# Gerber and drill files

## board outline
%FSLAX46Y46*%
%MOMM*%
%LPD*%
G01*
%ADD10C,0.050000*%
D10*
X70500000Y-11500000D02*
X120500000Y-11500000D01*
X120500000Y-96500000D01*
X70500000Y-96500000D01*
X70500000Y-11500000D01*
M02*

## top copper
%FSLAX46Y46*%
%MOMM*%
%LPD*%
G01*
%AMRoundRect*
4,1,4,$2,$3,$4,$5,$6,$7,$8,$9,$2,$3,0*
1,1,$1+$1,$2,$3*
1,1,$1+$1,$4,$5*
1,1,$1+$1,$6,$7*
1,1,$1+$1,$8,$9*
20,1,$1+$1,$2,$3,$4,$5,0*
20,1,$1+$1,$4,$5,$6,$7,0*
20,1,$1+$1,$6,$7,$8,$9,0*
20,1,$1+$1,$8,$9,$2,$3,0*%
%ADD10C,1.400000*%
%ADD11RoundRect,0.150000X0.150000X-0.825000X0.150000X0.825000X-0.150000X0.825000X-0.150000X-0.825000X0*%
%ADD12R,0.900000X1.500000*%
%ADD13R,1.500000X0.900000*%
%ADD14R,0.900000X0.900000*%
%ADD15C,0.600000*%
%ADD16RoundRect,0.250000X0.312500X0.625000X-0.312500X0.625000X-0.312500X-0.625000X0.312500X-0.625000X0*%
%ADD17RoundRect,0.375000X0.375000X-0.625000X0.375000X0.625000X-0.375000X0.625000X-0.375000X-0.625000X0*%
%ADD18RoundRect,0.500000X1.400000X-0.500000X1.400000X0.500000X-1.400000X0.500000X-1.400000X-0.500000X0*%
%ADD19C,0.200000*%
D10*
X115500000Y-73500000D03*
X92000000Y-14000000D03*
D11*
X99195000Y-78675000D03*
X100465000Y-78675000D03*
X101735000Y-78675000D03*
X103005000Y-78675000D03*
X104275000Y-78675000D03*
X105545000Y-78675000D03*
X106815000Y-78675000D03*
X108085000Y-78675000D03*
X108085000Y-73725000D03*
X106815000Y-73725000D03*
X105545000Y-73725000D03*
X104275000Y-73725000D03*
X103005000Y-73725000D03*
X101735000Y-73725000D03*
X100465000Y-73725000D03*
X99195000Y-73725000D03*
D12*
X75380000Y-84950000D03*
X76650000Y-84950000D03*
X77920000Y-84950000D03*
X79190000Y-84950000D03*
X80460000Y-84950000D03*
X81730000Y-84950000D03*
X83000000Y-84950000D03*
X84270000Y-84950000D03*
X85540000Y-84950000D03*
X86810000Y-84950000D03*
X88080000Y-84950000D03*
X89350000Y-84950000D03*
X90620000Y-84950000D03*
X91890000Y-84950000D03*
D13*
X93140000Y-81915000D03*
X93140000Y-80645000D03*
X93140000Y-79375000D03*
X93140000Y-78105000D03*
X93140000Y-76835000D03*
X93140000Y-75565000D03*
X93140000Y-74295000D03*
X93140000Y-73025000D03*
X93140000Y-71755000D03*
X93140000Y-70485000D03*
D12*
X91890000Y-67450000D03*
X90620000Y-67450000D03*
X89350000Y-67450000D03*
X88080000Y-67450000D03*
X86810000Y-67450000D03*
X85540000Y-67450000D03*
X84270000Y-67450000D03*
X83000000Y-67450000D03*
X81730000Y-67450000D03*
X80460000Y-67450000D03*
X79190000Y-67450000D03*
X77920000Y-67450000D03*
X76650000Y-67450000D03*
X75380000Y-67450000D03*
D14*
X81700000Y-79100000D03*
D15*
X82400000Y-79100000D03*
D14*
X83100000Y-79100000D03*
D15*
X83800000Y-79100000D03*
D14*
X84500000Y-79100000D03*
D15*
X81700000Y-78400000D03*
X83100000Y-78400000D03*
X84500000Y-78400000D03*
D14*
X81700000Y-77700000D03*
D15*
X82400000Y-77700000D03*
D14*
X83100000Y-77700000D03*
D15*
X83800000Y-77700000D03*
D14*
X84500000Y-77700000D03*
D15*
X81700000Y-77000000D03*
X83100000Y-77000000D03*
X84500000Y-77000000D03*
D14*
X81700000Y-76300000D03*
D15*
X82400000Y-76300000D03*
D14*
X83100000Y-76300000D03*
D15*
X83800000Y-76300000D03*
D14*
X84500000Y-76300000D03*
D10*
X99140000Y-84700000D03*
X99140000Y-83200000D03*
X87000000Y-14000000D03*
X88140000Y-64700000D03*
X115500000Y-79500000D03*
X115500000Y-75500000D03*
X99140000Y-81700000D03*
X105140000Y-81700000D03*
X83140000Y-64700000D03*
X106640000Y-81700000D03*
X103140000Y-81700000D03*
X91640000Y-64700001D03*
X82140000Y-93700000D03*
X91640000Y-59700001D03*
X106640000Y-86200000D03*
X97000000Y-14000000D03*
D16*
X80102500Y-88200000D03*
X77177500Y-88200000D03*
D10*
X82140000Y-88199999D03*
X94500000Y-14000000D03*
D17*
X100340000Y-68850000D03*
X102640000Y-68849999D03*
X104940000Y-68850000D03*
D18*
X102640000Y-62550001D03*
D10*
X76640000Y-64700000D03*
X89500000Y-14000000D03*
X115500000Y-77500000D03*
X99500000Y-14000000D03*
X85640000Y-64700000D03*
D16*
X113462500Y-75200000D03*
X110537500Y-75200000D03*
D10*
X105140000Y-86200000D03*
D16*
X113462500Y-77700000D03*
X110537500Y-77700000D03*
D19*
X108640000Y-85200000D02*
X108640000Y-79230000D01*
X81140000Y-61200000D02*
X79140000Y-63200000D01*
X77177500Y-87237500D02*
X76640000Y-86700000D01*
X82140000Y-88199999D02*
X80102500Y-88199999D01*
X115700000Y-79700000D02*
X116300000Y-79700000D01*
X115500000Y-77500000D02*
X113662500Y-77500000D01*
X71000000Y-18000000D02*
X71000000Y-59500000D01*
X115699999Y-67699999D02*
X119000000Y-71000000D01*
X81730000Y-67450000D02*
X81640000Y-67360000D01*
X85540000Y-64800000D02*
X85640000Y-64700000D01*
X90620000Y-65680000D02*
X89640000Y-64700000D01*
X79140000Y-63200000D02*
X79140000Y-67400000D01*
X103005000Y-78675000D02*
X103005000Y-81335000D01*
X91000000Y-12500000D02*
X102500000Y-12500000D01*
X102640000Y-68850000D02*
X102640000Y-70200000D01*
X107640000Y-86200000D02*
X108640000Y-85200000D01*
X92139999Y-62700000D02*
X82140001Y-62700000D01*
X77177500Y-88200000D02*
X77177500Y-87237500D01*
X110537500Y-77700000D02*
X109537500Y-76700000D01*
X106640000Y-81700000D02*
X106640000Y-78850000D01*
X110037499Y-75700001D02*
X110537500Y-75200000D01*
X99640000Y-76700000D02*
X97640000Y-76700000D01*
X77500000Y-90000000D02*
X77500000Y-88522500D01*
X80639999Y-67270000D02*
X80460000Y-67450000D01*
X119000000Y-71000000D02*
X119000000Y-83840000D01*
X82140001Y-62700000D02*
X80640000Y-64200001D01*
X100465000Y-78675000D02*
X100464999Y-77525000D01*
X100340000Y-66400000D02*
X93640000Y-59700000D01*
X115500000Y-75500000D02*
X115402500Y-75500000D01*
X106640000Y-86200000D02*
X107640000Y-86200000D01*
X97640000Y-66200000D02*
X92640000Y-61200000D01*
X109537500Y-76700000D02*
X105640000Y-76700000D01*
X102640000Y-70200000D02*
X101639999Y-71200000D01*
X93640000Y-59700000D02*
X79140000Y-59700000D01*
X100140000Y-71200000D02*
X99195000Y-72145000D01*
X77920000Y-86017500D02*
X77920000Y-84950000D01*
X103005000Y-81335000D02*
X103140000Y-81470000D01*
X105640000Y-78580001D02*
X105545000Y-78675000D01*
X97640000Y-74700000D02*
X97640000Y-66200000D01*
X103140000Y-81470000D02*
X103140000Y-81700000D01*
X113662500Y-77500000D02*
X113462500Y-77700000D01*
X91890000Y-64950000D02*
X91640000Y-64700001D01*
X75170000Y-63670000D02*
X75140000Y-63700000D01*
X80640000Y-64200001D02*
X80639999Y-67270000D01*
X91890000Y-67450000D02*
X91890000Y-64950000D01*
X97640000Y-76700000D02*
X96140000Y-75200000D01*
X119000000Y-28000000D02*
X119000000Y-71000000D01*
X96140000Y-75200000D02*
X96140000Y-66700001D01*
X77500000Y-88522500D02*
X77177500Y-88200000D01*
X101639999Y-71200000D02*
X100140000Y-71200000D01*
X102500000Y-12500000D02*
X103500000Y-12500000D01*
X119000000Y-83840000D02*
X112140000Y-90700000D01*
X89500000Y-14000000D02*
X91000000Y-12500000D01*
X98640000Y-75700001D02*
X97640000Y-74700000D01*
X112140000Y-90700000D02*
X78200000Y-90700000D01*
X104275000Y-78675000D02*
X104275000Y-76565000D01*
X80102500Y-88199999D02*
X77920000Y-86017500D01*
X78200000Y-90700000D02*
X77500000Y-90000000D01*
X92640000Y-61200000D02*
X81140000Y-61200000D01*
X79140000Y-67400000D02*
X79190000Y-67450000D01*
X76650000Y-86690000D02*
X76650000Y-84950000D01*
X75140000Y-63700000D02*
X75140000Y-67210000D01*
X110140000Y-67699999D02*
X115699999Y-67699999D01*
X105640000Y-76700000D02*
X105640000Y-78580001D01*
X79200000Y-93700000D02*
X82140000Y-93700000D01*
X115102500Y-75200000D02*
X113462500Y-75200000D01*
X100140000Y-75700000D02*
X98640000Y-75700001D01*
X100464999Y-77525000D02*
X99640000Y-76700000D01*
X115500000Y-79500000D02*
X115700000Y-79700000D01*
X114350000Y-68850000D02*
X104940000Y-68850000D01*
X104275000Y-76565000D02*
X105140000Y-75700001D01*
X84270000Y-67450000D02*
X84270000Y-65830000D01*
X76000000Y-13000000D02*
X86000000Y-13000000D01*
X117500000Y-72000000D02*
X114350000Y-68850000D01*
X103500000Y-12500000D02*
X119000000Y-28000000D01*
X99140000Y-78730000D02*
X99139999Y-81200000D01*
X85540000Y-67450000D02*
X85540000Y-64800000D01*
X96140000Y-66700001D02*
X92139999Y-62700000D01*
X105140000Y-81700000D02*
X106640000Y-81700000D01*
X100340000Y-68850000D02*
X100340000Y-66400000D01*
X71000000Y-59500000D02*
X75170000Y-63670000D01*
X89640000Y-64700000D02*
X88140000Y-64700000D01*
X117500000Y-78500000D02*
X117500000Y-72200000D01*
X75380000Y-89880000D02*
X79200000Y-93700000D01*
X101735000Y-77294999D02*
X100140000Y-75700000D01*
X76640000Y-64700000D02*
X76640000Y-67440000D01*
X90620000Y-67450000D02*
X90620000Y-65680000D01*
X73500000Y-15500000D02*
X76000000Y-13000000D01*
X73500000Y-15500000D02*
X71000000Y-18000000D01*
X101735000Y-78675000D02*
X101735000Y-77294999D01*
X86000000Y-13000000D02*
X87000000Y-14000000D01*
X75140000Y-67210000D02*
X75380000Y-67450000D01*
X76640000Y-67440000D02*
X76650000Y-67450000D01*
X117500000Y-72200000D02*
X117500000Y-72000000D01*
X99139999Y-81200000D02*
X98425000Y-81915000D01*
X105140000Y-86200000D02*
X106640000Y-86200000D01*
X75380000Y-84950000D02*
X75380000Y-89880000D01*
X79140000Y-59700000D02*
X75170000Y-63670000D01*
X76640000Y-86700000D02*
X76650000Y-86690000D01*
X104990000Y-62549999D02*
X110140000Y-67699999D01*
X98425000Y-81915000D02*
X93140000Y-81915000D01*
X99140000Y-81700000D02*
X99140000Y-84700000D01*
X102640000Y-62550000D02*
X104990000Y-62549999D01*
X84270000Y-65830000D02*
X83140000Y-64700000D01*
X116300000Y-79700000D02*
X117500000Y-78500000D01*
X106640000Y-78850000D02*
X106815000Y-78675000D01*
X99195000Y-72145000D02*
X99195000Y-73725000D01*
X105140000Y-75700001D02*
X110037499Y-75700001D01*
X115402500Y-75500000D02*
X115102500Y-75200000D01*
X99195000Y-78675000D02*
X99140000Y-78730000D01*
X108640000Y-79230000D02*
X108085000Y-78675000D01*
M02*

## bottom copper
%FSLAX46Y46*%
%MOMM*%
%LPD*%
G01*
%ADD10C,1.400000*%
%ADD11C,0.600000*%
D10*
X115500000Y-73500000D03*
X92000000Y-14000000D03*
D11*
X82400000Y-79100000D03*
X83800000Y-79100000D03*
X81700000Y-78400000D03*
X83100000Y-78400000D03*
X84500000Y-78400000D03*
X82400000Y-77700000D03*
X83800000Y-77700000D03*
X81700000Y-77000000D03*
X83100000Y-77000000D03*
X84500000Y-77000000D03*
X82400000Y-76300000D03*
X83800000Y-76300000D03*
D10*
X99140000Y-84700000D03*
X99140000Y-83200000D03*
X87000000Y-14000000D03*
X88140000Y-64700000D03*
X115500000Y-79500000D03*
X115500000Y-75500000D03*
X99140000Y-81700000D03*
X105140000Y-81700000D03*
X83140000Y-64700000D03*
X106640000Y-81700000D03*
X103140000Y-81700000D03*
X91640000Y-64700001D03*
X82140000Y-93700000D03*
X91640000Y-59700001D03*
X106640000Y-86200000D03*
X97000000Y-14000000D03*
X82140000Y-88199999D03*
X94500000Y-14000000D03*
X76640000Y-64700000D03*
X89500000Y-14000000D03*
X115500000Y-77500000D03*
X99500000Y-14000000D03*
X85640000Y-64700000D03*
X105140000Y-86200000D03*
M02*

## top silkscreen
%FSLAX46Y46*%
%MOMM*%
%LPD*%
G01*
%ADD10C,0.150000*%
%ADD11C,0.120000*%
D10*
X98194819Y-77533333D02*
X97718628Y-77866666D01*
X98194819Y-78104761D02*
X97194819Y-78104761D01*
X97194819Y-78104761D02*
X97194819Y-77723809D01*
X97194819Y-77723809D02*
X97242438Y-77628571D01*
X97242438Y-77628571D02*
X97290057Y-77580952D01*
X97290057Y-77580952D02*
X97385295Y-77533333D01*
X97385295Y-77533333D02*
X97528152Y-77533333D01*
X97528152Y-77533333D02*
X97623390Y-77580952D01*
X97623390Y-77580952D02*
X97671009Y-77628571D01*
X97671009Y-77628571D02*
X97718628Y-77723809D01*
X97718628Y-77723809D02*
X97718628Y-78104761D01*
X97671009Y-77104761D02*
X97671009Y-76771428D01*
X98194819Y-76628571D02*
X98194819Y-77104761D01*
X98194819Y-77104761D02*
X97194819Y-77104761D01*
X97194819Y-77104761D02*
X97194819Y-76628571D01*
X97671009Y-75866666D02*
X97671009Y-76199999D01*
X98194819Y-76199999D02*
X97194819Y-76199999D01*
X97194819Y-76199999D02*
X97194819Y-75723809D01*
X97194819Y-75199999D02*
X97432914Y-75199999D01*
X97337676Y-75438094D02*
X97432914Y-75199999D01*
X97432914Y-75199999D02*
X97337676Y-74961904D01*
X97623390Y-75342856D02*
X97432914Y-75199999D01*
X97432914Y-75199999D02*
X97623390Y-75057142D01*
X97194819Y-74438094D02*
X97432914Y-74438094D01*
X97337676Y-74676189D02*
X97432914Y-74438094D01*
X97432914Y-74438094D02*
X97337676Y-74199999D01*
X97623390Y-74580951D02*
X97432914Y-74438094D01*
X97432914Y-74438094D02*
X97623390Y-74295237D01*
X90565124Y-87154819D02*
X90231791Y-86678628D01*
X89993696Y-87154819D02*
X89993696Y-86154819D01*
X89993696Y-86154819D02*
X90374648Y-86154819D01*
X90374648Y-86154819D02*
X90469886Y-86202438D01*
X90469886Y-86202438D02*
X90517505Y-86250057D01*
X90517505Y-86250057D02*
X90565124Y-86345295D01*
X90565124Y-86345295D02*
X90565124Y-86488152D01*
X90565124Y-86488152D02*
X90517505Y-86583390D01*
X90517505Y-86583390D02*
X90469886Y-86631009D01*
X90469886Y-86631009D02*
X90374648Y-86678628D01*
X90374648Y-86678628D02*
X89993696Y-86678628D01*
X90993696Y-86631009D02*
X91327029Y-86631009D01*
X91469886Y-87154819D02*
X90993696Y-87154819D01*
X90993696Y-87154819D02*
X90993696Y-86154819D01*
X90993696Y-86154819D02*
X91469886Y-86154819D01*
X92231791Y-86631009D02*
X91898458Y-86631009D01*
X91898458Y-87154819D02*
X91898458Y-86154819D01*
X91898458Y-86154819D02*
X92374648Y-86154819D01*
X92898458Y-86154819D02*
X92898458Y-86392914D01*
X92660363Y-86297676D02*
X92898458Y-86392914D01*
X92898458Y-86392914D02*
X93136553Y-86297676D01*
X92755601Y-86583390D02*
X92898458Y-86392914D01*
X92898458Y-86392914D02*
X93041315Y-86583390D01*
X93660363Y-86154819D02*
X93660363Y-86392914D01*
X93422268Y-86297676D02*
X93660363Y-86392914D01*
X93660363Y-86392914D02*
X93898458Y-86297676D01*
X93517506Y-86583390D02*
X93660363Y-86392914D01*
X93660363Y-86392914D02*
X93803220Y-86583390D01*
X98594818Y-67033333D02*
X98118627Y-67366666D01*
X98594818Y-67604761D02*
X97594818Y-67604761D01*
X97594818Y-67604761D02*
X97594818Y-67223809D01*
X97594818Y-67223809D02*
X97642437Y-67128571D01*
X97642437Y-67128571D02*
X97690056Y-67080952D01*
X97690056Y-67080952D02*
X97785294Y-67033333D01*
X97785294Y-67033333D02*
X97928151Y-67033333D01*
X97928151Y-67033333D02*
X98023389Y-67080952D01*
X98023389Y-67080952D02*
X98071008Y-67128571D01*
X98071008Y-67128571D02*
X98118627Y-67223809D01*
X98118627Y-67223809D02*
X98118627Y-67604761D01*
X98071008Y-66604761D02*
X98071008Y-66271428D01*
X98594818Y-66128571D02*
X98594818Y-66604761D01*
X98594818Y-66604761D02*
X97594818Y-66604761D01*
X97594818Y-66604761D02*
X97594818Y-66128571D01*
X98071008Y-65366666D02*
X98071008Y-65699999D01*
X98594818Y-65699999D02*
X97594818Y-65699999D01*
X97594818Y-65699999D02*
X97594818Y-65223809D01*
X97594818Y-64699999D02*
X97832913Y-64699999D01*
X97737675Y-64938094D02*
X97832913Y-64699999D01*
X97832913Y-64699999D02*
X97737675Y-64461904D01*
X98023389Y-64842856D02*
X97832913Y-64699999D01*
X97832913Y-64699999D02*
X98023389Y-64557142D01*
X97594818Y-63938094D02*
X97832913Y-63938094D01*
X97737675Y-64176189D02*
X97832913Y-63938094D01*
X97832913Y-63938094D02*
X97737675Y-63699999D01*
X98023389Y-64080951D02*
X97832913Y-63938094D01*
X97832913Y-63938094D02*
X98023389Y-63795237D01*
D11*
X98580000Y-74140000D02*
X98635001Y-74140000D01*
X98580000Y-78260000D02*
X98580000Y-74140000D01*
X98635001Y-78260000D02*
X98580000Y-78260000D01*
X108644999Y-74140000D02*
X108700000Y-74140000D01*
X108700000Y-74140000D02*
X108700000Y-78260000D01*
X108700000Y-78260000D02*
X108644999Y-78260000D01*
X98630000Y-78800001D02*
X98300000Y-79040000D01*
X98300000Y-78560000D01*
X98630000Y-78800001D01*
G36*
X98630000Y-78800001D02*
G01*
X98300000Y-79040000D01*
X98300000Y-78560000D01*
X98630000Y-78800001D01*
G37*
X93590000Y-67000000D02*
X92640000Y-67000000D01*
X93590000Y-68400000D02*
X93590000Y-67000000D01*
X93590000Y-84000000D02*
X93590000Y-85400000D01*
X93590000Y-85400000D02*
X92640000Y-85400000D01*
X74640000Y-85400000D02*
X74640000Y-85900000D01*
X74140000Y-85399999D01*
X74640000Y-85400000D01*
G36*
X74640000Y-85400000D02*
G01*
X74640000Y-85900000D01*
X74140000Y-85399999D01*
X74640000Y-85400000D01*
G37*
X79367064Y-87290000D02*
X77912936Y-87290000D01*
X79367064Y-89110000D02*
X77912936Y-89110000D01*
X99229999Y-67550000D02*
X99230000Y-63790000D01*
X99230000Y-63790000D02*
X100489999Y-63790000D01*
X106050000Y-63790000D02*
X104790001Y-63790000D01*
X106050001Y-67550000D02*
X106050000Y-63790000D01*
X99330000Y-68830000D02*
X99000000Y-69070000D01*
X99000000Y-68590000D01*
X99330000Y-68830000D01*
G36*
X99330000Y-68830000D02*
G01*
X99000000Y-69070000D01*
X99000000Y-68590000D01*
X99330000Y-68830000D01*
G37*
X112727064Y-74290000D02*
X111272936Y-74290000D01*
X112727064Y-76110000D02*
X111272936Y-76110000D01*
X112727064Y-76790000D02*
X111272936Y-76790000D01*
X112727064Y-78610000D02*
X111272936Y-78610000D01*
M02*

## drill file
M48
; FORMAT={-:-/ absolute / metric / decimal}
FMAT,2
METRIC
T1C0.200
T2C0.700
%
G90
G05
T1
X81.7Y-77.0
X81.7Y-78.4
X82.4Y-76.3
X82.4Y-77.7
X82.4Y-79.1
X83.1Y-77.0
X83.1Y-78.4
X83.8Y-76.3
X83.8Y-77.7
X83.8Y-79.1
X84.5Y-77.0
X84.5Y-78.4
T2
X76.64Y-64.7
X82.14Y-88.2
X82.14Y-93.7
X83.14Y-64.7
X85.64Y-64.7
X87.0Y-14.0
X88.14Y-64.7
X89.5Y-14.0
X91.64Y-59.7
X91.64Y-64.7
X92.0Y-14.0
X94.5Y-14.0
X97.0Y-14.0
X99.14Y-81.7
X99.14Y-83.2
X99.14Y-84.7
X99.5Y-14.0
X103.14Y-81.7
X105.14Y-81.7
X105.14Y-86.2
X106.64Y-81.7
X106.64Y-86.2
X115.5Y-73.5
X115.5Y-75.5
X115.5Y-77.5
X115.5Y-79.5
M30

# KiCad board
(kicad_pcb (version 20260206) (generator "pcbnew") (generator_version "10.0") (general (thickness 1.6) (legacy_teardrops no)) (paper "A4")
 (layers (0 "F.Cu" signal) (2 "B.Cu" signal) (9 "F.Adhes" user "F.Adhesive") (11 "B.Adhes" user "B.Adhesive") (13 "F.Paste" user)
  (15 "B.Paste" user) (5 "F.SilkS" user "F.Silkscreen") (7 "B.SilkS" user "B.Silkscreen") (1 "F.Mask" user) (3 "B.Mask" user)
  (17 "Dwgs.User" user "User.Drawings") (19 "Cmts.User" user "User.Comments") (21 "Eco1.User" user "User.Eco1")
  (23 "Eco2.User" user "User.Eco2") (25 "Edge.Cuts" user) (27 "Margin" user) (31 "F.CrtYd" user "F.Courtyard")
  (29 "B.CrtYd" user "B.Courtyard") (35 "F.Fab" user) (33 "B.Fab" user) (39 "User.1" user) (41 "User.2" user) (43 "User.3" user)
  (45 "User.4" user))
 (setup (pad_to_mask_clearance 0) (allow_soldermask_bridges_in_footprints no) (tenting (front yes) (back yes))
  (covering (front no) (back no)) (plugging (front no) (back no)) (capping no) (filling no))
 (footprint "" (layer "F.Cu") (at 115.5 73.5 90)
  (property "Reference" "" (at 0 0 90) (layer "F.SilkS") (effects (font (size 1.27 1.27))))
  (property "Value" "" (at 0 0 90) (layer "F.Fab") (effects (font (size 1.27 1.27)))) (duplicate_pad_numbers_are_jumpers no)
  (pad "4" thru_hole circle (at 0 0 90) (size 1.4 1.4) (drill 0.7) (layers "*.Cu" "*.Mask") (remove_unused_layers no)))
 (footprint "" (layer "F.Cu") (at 92 14)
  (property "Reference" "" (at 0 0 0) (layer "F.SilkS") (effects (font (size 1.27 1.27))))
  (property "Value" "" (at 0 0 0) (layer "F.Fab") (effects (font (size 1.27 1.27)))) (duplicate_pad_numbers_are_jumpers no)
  (pad "4" thru_hole circle (at 0 0) (size 1.4 1.4) (drill 0.7) (layers "*.Cu" "*.Mask") (remove_unused_layers no)))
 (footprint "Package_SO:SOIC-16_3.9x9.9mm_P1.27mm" (layer "F.Cu") (at 103.64 76.2 90)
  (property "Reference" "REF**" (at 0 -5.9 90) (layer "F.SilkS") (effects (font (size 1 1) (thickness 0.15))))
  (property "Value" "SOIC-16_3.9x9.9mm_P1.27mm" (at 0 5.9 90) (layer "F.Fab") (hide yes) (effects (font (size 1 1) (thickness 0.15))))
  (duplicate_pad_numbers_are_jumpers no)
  (fp_line (start 2.06 -5.06) (end 2.06 -5.004999) (stroke (width 0.12) (type solid)) (layer "F.SilkS"))
  (fp_line (start -2.06 -5.06) (end 2.06 -5.06) (stroke (width 0.12) (type solid)) (layer "F.SilkS"))
  (fp_line (start -2.06 -5.004999) (end -2.06 -5.06) (stroke (width 0.12) (type solid)) (layer "F.SilkS"))
  (fp_line (start 2.06 5.004999) (end 2.06 5.06) (stroke (width 0.12) (type solid)) (layer "F.SilkS"))
  (fp_line (start 2.06 5.06) (end -2.06 5.06) (stroke (width 0.12) (type solid)) (layer "F.SilkS"))
  (fp_line (start -2.06 5.06) (end -2.06 5.004999) (stroke (width 0.12) (type solid)) (layer "F.SilkS"))
  (fp_poly (pts (xy -2.600001 -5.01) (xy -2.84 -5.34) (xy -2.36 -5.34)) (stroke (width 0.12) (type solid)) (fill yes) (layer "F.SilkS"))
  (pad "1" smd roundrect (at -2.475 -4.445 90) (size 1.95 0.6) (layers "F.Cu" "F.Mask" "F.Paste") (roundrect_rratio 0.25))
  (pad "2" smd roundrect (at -2.475 -3.175 90) (size 1.95 0.6) (layers "F.Cu" "F.Mask" "F.Paste") (roundrect_rratio 0.25))
  (pad "3" smd roundrect (at -2.475 -1.905 90) (size 1.95 0.6) (layers "F.Cu" "F.Mask" "F.Paste") (roundrect_rratio 0.25))
  (pad "4" smd roundrect (at -2.475 -0.635 90) (size 1.95 0.6) (layers "F.Cu" "F.Mask" "F.Paste") (roundrect_rratio 0.25))
  (pad "5" smd roundrect (at -2.475 0.635 90) (size 1.95 0.6) (layers "F.Cu" "F.Mask" "F.Paste") (roundrect_rratio 0.25))
  (pad "6" smd roundrect (at -2.475 1.905 90) (size 1.95 0.6) (layers "F.Cu" "F.Mask" "F.Paste") (roundrect_rratio 0.25))
  (pad "7" smd roundrect (at -2.475 3.175 90) (size 1.95 0.6) (layers "F.Cu" "F.Mask" "F.Paste") (roundrect_rratio 0.25))
  (pad "8" smd roundrect (at -2.475 4.445 90) (size 1.95 0.6) (layers "F.Cu" "F.Mask" "F.Paste") (roundrect_rratio 0.25))
  (pad "9" smd roundrect (at 2.475 4.445 90) (size 1.95 0.6) (layers "F.Cu" "F.Mask" "F.Paste") (roundrect_rratio 0.25))
  (pad "10" smd roundrect (at 2.475 3.175 90) (size 1.95 0.6) (layers "F.Cu" "F.Mask" "F.Paste") (roundrect_rratio 0.25))
  (pad "11" smd roundrect (at 2.475 1.905 90) (size 1.95 0.6) (layers "F.Cu" "F.Mask" "F.Paste") (roundrect_rratio 0.25))
  (pad "12" smd roundrect (at 2.475 0.635 90) (size 1.95 0.6) (layers "F.Cu" "F.Mask" "F.Paste") (roundrect_rratio 0.25))
  (pad "13" smd roundrect (at 2.475 -0.635 90) (size 1.95 0.6) (layers "F.Cu" "F.Mask" "F.Paste") (roundrect_rratio 0.25))
  (pad "14" smd roundrect (at 2.475 -1.905 90) (size 1.95 0.6) (layers "F.Cu" "F.Mask" "F.Paste") (roundrect_rratio 0.25))
  (pad "15" smd roundrect (at 2.475 -3.175 90) (size 1.95 0.6) (layers "F.Cu" "F.Mask" "F.Paste") (roundrect_rratio 0.25))
  (pad "16" smd roundrect (at 2.475 -4.445 90) (size 1.95 0.6) (layers "F.Cu" "F.Mask" "F.Paste") (roundrect_rratio 0.25)))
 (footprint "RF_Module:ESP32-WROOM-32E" (layer "F.Cu") (at 80.64 76.2 90)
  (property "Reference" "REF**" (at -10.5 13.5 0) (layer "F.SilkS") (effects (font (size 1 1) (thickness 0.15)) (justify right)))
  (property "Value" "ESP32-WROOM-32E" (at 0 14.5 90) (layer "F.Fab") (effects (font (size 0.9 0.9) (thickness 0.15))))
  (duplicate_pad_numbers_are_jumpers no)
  (fp_line (start 9.2 12.95) (end 9.2 12) (stroke (width 0.12) (type solid)) (layer "F.SilkS"))
  (fp_line (start 7.8 12.95) (end 9.2 12.95) (stroke (width 0.12) (type solid)) (layer "F.SilkS"))
  (fp_line (start -7.8 12.95) (end -9.2 12.95) (stroke (width 0.12) (type solid)) (layer "F.SilkS"))
  (fp_line (start -9.2 12.95) (end -9.2 12) (stroke (width 0.12) (type solid)) (layer "F.SilkS"))
  (fp_poly (pts (xy -9.2 -6) (xy -9.7 -6) (xy -9.199999 -6.5) (xy -9.2 -6)) (stroke (width 0.12) (type solid)) (fill yes) (layer "F.SilkS"))
  (pad "1" smd rect (at -8.75 -5.26 90) (size 1.5 0.9) (layers "F.Cu" "F.Mask" "F.Paste"))
  (pad "2" smd rect (at -8.75 -3.99 90) (size 1.5 0.9) (layers "F.Cu" "F.Mask" "F.Paste"))
  (pad "3" smd rect (at -8.75 -2.72 90) (size 1.5 0.9) (layers "F.Cu" "F.Mask" "F.Paste"))
  (pad "4" smd rect (at -8.75 -1.45 90) (size 1.5 0.9) (layers "F.Cu" "F.Mask" "F.Paste"))
  (pad "5" smd rect (at -8.75 -0.18 90) (size 1.5 0.9) (layers "F.Cu" "F.Mask" "F.Paste"))
  (pad "6" smd rect (at -8.75 1.09 90) (size 1.5 0.9) (layers "F.Cu" "F.Mask" "F.Paste"))
  (pad "7" smd rect (at -8.75 2.36 90) (size 1.5 0.9) (layers "F.Cu" "F.Mask" "F.Paste"))
  (pad "8" smd rect (at -8.75 3.63 90) (size 1.5 0.9) (layers "F.Cu" "F.Mask" "F.Paste"))
  (pad "9" smd rect (at -8.75 4.9 90) (size 1.5 0.9) (layers "F.Cu" "F.Mask" "F.Paste"))
  (pad "10" smd rect (at -8.75 6.17 90) (size 1.5 0.9) (layers "F.Cu" "F.Mask" "F.Paste"))
  (pad "11" smd rect (at -8.75 7.44 90) (size 1.5 0.9) (layers "F.Cu" "F.Mask" "F.Paste"))
  (pad "12" smd rect (at -8.75 8.71 90) (size 1.5 0.9) (layers "F.Cu" "F.Mask" "F.Paste"))
  (pad "13" smd rect (at -8.75 9.98 90) (size 1.5 0.9) (layers "F.Cu" "F.Mask" "F.Paste"))
  (pad "14" smd rect (at -8.75 11.25 90) (size 1.5 0.9) (layers "F.Cu" "F.Mask" "F.Paste"))
  (pad "15" smd rect (at -5.715 12.5 180) (size 1.5 0.9) (layers "F.Cu" "F.Mask" "F.Paste"))
  (pad "16" smd rect (at -4.445 12.5 180) (size 1.5 0.9) (layers "F.Cu" "F.Mask" "F.Paste"))
  (pad "17" smd rect (at -3.175 12.5 180) (size 1.5 0.9) (layers "F.Cu" "F.Mask" "F.Paste"))
  (pad "18" smd rect (at -1.905 12.5 180) (size 1.5 0.9) (layers "F.Cu" "F.Mask" "F.Paste"))
  (pad "19" smd rect (at -0.635 12.5 180) (size 1.5 0.9) (layers "F.Cu" "F.Mask" "F.Paste"))
  (pad "20" smd rect (at 0.635 12.5 180) (size 1.5 0.9) (layers "F.Cu" "F.Mask" "F.Paste"))
  (pad "21" smd rect (at 1.905 12.5 180) (size 1.5 0.9) (layers "F.Cu" "F.Mask" "F.Paste"))
  (pad "22" smd rect (at 3.175 12.5 180) (size 1.5 0.9) (layers "F.Cu" "F.Mask" "F.Paste"))
  (pad "23" smd rect (at 4.445 12.5 180) (size 1.5 0.9) (layers "F.Cu" "F.Mask" "F.Paste"))
  (pad "24" smd rect (at 5.715 12.5 180) (size 1.5 0.9) (layers "F.Cu" "F.Mask" "F.Paste"))
  (pad "25" smd rect (at 8.75 11.25 90) (size 1.5 0.9) (layers "F.Cu" "F.Mask" "F.Paste"))
  (pad "26" smd rect (at 8.75 9.98 90) (size 1.5 0.9) (layers "F.Cu" "F.Mask" "F.Paste"))
  (pad "27" smd rect (at 8.75 8.71 90) (size 1.5 0.9) (layers "F.Cu" "F.Mask" "F.Paste"))
  (pad "28" smd rect (at 8.75 7.44 90) (size 1.5 0.9) (layers "F.Cu" "F.Mask" "F.Paste"))
  (pad "29" smd rect (at 8.75 6.17 90) (size 1.5 0.9) (layers "F.Cu" "F.Mask" "F.Paste"))
  (pad "30" smd rect (at 8.75 4.9 90) (size 1.5 0.9) (layers "F.Cu" "F.Mask" "F.Paste"))
  (pad "31" smd rect (at 8.75 3.63 90) (size 1.5 0.9) (layers "F.Cu" "F.Mask" "F.Paste"))
  (pad "32" smd rect (at 8.75 2.36 90) (size 1.5 0.9) (layers "F.Cu" "F.Mask" "F.Paste"))
  (pad "33" smd rect (at 8.75 1.09 90) (size 1.5 0.9) (layers "F.Cu" "F.Mask" "F.Paste"))
  (pad "34" smd rect (at 8.75 -0.18 90) (size 1.5 0.9) (layers "F.Cu" "F.Mask" "F.Paste"))
  (pad "35" smd rect (at 8.75 -1.45 90) (size 1.5 0.9) (layers "F.Cu" "F.Mask" "F.Paste"))
  (pad "36" smd rect (at 8.75 -2.72 90) (size 1.5 0.9) (layers "F.Cu" "F.Mask" "F.Paste"))
  (pad "37" smd rect (at 8.75 -3.99 90) (size 1.5 0.9) (layers "F.Cu" "F.Mask" "F.Paste"))
  (pad "38" smd rect (at 8.75 -5.26 90) (size 1.5 0.9) (layers "F.Cu" "F.Mask" "F.Paste"))
  (pad "39" smd rect (at -2.9 1.06 90) (size 0.9 0.9) (layers "F.Cu" "F.Mask" "F.Paste") (zone_connect 2))
  (pad "39" thru_hole circle (at -2.9 1.76 90) (size 0.6 0.6) (drill 0.2) (layers "*.Cu" "*.Mask") (remove_unused_layers no)
   (zone_connect 2))
  (pad "39" smd rect (at -2.9 2.46 90) (size 0.9 0.9) (layers "F.Cu" "F.Mask" "F.Paste") (zone_connect 2))
  (pad "39" thru_hole circle (at -2.9 3.16 90) (size 0.6 0.6) (drill 0.2) (layers "*.Cu" "*.Mask") (remove_unused_layers no)
   (zone_connect 2))
  (pad "39" smd rect (at -2.9 3.86 90) (size 0.9 0.9) (layers "F.Cu" "F.Mask" "F.Paste") (zone_connect 2))
  (pad "39" thru_hole circle (at -2.2 1.06 90) (size 0.6 0.6) (drill 0.2) (layers "*.Cu" "*.Mask") (remove_unused_layers no)
   (zone_connect 2))
  (pad "39" thru_hole circle (at -2.2 2.46 90) (size 0.6 0.6) (drill 0.2) (layers "*.Cu" "*.Mask") (remove_unused_layers no)
   (zone_connect 2))
  (pad "39" thru_hole circle (at -2.2 3.86 90) (size 0.6 0.6) (drill 0.2) (layers "*.Cu" "*.Mask") (remove_unused_layers no)
   (zone_connect 2))
  (pad "39" smd rect (at -1.5 1.06 90) (size 0.9 0.9) (layers "F.Cu" "F.Mask" "F.Paste") (zone_connect 2))
  (pad "39" thru_hole circle (at -1.5 1.76 90) (size 0.6 0.6) (drill 0.2) (layers "*.Cu" "*.Mask") (remove_unused_layers no)
   (zone_connect 2))
  (pad "39" smd rect (at -1.5 2.46 90) (size 0.9 0.9) (layers "F.Cu" "F.Mask" "F.Paste") (zone_connect 2))
  (pad "39" thru_hole circle (at -1.5 3.16 90) (size 0.6 0.6) (drill 0.2) (layers "*.Cu" "*.Mask") (remove_unused_layers no)
   (zone_connect 2))
  (pad "39" smd rect (at -1.5 3.86 90) (size 0.9 0.9) (layers "F.Cu" "F.Mask" "F.Paste") (zone_connect 2))
  (pad "39" thru_hole circle (at -0.8 1.06 90) (size 0.6 0.6) (drill 0.2) (layers "*.Cu" "*.Mask") (remove_unused_layers no)
   (zone_connect 2))
  (pad "39" thru_hole circle (at -0.8 2.46 90) (size 0.6 0.6) (drill 0.2) (layers "*.Cu" "*.Mask") (remove_unused_layers no)
   (zone_connect 2))
  (pad "39" thru_hole circle (at -0.8 3.86 90) (size 0.6 0.6) (drill 0.2) (layers "*.Cu" "*.Mask") (remove_unused_layers no)
   (zone_connect 2))
  (pad "39" smd rect (at -0.1 1.06 90) (size 0.9 0.9) (layers "F.Cu" "F.Mask" "F.Paste") (zone_connect 2))
  (pad "39" thru_hole circle (at -0.1 1.76 90) (size 0.6 0.6) (drill 0.2) (layers "*.Cu" "*.Mask") (remove_unused_layers no)
   (zone_connect 2))
  (pad "39" smd rect (at -0.1 2.46 90) (size 0.9 0.9) (layers "F.Cu" "F.Mask" "F.Paste") (zone_connect 2))
  (pad "39" thru_hole circle (at -0.1 3.16 90) (size 0.6 0.6) (drill 0.2) (layers "*.Cu" "*.Mask") (remove_unused_layers no)
   (zone_connect 2))
  (pad "39" smd rect (at -0.1 3.86 90) (size 0.9 0.9) (layers "F.Cu" "F.Mask" "F.Paste") (zone_connect 2))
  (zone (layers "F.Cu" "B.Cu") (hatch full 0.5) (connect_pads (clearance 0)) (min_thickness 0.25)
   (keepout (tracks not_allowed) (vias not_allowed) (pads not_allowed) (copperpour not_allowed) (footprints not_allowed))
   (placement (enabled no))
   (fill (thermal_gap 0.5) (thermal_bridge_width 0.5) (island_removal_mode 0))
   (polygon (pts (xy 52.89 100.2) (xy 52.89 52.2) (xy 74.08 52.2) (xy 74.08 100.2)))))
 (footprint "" (layer "F.Cu") (at 99.14 84.7 90)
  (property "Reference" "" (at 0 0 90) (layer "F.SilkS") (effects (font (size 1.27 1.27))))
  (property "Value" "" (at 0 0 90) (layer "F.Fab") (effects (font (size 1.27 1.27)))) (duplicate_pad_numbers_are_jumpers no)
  (pad "4" thru_hole circle (at 0 0 90) (size 1.4 1.4) (drill 0.7) (layers "*.Cu" "*.Mask") (remove_unused_layers no)))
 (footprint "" (layer "F.Cu") (at 99.14 83.2 90)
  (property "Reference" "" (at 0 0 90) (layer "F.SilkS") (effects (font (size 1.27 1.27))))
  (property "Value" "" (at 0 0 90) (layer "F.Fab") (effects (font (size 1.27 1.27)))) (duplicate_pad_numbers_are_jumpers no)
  (pad "4" thru_hole circle (at 0 0 90) (size 1.4 1.4) (drill 0.7) (layers "*.Cu" "*.Mask") (remove_unused_layers no)))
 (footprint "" (layer "F.Cu") (at 87 14)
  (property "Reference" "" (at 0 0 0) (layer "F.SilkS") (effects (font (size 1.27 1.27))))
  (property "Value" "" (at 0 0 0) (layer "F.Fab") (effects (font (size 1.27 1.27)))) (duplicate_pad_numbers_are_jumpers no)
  (pad "4" thru_hole circle (at 0 0) (size 1.4 1.4) (drill 0.7) (layers "*.Cu" "*.Mask") (remove_unused_layers no)))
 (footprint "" (layer "F.Cu") (at 88.14 64.7 90)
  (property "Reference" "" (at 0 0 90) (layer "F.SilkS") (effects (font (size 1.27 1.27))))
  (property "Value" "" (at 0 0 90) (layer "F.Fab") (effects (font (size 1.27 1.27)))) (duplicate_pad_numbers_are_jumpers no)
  (pad "4" thru_hole circle (at 0 0 90) (size 1.4 1.4) (drill 0.7) (layers "*.Cu" "*.Mask") (remove_unused_layers no)))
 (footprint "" (layer "F.Cu") (at 115.5 79.5 90)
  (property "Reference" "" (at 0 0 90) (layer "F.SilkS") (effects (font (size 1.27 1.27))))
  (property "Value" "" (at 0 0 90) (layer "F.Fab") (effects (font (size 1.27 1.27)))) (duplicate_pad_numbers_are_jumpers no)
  (pad "4" thru_hole circle (at 0 0 90) (size 1.4 1.4) (drill 0.7) (layers "*.Cu" "*.Mask") (remove_unused_layers no)))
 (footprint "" (layer "F.Cu") (at 115.5 75.5 90)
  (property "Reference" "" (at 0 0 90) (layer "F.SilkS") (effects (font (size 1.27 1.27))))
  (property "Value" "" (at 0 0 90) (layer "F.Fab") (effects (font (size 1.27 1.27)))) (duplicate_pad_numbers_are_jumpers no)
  (pad "4" thru_hole circle (at 0 0 90) (size 1.4 1.4) (drill 0.7) (layers "*.Cu" "*.Mask") (remove_unused_layers no)))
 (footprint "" (layer "F.Cu") (at 99.14 81.7 90)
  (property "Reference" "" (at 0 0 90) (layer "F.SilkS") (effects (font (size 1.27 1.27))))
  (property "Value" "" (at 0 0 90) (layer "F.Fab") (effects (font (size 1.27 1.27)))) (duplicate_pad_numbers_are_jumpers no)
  (pad "4" thru_hole circle (at 0 0 90) (size 1.4 1.4) (drill 0.7) (layers "*.Cu" "*.Mask") (remove_unused_layers no)))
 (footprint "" (layer "F.Cu") (at 105.14 81.7 90)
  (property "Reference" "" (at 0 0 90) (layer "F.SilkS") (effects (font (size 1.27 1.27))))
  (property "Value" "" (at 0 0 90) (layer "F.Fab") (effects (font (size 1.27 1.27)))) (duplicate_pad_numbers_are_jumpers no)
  (pad "4" thru_hole circle (at 0 0 90) (size 1.4 1.4) (drill 0.7) (layers "*.Cu" "*.Mask") (remove_unused_layers no)))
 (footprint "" (layer "F.Cu") (at 83.14 64.7 90)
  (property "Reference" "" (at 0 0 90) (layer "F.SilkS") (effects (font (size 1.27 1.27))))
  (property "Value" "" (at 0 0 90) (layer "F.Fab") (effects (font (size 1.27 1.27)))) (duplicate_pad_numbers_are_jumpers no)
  (pad "4" thru_hole circle (at 0 0 90) (size 1.4 1.4) (drill 0.7) (layers "*.Cu" "*.Mask") (remove_unused_layers no)))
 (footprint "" (layer "F.Cu") (at 106.64 81.7 90)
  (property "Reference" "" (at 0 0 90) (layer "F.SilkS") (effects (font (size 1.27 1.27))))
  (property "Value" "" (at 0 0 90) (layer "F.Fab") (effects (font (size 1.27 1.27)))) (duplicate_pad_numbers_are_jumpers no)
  (pad "4" thru_hole circle (at 0 0 90) (size 1.4 1.4) (drill 0.7) (layers "*.Cu" "*.Mask") (remove_unused_layers no)))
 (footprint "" (layer "F.Cu") (at 103.14 81.7 90)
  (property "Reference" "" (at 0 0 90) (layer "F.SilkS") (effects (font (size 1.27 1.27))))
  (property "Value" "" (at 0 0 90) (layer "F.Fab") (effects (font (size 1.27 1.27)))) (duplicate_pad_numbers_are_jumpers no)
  (pad "4" thru_hole circle (at 0 0 90) (size 1.4 1.4) (drill 0.7) (layers "*.Cu" "*.Mask") (remove_unused_layers no)))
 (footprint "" (layer "F.Cu") (at 91.64 64.700001 90)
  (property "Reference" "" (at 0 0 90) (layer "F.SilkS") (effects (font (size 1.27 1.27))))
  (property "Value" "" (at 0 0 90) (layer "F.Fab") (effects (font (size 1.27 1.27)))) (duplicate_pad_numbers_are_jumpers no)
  (pad "4" thru_hole circle (at 0 0 90) (size 1.4 1.4) (drill 0.7) (layers "*.Cu" "*.Mask") (remove_unused_layers no)))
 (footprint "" (layer "F.Cu") (at 82.14 93.7 90)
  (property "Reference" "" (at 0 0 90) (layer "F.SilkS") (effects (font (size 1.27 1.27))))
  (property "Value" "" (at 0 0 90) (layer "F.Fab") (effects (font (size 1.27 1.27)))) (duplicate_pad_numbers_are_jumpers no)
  (pad "4" thru_hole circle (at 0 0 90) (size 1.4 1.4) (drill 0.7) (layers "*.Cu" "*.Mask") (remove_unused_layers no)))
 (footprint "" (layer "F.Cu") (at 91.64 59.700001 90)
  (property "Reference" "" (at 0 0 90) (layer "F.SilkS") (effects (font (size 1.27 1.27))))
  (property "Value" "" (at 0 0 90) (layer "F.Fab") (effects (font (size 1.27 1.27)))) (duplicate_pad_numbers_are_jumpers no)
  (pad "4" thru_hole circle (at 0 0 90) (size 1.4 1.4) (drill 0.7) (layers "*.Cu" "*.Mask") (remove_unused_layers no)))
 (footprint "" (layer "F.Cu") (at 106.64 86.2 90)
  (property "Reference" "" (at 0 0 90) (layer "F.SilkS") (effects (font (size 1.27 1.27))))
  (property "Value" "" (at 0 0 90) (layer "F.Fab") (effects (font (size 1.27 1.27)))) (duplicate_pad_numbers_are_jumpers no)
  (pad "4" thru_hole circle (at 0 0 90) (size 1.4 1.4) (drill 0.7) (layers "*.Cu" "*.Mask") (remove_unused_layers no)))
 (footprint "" (layer "F.Cu") (at 97 14)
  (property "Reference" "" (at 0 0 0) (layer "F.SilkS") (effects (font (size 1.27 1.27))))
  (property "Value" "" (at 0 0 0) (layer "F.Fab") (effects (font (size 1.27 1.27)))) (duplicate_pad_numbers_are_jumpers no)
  (pad "4" thru_hole circle (at 0 0) (size 1.4 1.4) (drill 0.7) (layers "*.Cu" "*.Mask") (remove_unused_layers no)))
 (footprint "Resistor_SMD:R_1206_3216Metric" (layer "F.Cu") (at 78.64 88.2 180)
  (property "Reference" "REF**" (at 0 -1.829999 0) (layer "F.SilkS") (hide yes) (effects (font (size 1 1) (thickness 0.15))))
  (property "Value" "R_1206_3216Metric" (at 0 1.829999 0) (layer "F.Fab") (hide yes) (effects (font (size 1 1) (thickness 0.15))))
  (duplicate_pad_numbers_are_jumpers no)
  (fp_line (start -0.727064 0.91) (end 0.727064 0.91) (stroke (width 0.12) (type solid)) (layer "F.SilkS"))
  (fp_line (start -0.727064 -0.91) (end 0.727064 -0.91) (stroke (width 0.12) (type solid)) (layer "F.SilkS"))
  (pad "1" smd roundrect (at -1.4625 0 180) (size 1.125 1.75) (layers "F.Cu" "F.Mask" "F.Paste") (roundrect_rratio 0.222222))
  (pad "2" smd roundrect (at 1.4625 0 180) (size 1.125 1.75) (layers "F.Cu" "F.Mask" "F.Paste") (roundrect_rratio 0.222222)))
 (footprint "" (layer "F.Cu") (at 82.14 88.199999 90)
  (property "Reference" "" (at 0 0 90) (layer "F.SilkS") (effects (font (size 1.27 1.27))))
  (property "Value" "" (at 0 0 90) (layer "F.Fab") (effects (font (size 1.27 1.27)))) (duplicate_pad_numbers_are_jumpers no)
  (pad "4" thru_hole circle (at 0 0 90) (size 1.4 1.4) (drill 0.7) (layers "*.Cu" "*.Mask") (remove_unused_layers no)))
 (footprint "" (layer "F.Cu") (at 94.5 14)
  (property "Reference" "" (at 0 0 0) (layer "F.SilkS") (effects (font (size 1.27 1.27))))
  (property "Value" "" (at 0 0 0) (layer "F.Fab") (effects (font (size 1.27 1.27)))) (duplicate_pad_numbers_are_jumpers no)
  (pad "4" thru_hole circle (at 0 0) (size 1.4 1.4) (drill 0.7) (layers "*.Cu" "*.Mask") (remove_unused_layers no)))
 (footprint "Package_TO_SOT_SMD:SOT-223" (layer "F.Cu") (at 102.64 65.7 90)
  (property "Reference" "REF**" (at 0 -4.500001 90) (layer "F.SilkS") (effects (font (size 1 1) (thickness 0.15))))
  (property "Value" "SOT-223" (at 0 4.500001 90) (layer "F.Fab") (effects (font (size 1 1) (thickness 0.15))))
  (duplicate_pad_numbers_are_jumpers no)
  (fp_line (start -1.85 -3.410001) (end 1.91 -3.41) (stroke (width 0.12) (type solid)) (layer "F.SilkS"))
  (fp_line (start 1.91 -3.41) (end 1.91 -2.150001) (stroke (width 0.12) (type solid)) (layer "F.SilkS"))
  (fp_line (start 1.91 3.41) (end 1.91 2.150001) (stroke (width 0.12) (type solid)) (layer "F.SilkS"))
  (fp_line (start -1.85 3.410001) (end 1.91 3.41) (stroke (width 0.12) (type solid)) (layer "F.SilkS"))
  (fp_poly
   (pts (xy -3.13 -3.31) (xy -3.37 -3.64) (xy -2.89 -3.64) (xy -3.13 -3.31)) (stroke (width 0.12) (type solid)) (fill yes) (layer "F.SilkS"))
  (pad "1" smd roundrect (at -3.15 -2.3 90) (size 2 1.5) (layers "F.Cu" "F.Mask" "F.Paste") (roundrect_rratio 0.25))
  (pad "2" smd roundrect (at -3.149999 0 90) (size 2 1.5) (layers "F.Cu" "F.Mask" "F.Paste") (roundrect_rratio 0.25))
  (pad "3" smd roundrect (at -3.15 2.3 90) (size 2 1.5) (layers "F.Cu" "F.Mask" "F.Paste") (roundrect_rratio 0.25))
  (pad "4" smd roundrect (at 3.149999 0 90) (size 2 3.8) (layers "F.Cu" "F.Mask" "F.Paste") (roundrect_rratio 0.25)))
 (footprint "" (layer "F.Cu") (at 76.64 64.7 90)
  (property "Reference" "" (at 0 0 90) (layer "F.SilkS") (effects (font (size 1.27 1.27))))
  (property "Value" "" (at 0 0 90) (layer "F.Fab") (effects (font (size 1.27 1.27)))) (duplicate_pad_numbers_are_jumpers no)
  (pad "4" thru_hole circle (at 0 0 90) (size 1.4 1.4) (drill 0.7) (layers "*.Cu" "*.Mask") (remove_unused_layers no)))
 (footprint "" (layer "F.Cu") (at 89.5 14)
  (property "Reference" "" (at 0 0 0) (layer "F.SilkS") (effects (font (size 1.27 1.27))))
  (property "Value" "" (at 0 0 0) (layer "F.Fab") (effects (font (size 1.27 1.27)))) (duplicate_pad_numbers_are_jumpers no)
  (pad "4" thru_hole circle (at 0 0) (size 1.4 1.4) (drill 0.7) (layers "*.Cu" "*.Mask") (remove_unused_layers no)))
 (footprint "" (layer "F.Cu") (at 115.5 77.5 90)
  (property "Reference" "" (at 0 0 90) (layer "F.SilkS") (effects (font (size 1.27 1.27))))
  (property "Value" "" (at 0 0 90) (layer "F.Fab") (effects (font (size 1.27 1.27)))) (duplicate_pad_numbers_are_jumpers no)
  (pad "4" thru_hole circle (at 0 0 90) (size 1.4 1.4) (drill 0.7) (layers "*.Cu" "*.Mask") (remove_unused_layers no)))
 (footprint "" (layer "F.Cu") (at 99.5 14)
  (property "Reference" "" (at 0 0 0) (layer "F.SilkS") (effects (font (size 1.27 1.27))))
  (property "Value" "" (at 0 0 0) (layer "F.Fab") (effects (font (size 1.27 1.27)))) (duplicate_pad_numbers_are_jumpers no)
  (pad "4" thru_hole circle (at 0 0) (size 1.4 1.4) (drill 0.7) (layers "*.Cu" "*.Mask") (remove_unused_layers no)))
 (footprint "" (layer "F.Cu") (at 85.64 64.7 90)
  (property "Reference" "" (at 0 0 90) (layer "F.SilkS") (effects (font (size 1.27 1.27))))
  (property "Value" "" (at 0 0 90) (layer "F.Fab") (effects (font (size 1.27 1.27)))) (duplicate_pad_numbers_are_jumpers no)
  (pad "4" thru_hole circle (at 0 0 90) (size 1.4 1.4) (drill 0.7) (layers "*.Cu" "*.Mask") (remove_unused_layers no)))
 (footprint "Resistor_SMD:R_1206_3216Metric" (layer "F.Cu") (at 112 75.2 180)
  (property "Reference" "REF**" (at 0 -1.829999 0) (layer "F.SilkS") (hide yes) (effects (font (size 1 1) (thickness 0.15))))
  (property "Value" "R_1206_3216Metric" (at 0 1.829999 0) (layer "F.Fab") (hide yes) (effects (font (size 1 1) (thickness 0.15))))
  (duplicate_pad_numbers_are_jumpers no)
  (fp_line (start -0.727064 0.91) (end 0.727064 0.91) (stroke (width 0.12) (type solid)) (layer "F.SilkS"))
  (fp_line (start -0.727064 -0.91) (end 0.727064 -0.91) (stroke (width 0.12) (type solid)) (layer "F.SilkS"))
  (pad "1" smd roundrect (at -1.4625 0 180) (size 1.125 1.75) (layers "F.Cu" "F.Mask" "F.Paste") (roundrect_rratio 0.222222))
  (pad "2" smd roundrect (at 1.4625 0 180) (size 1.125 1.75) (layers "F.Cu" "F.Mask" "F.Paste") (roundrect_rratio 0.222222)))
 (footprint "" (layer "F.Cu") (at 105.14 86.2 90)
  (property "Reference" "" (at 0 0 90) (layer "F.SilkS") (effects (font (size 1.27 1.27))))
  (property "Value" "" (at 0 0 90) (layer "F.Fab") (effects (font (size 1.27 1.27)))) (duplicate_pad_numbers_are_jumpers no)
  (pad "4" thru_hole circle (at 0 0 90) (size 1.4 1.4) (drill 0.7) (layers "*.Cu" "*.Mask") (remove_unused_layers no)))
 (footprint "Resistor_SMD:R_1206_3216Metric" (layer "F.Cu") (at 112 77.7 180)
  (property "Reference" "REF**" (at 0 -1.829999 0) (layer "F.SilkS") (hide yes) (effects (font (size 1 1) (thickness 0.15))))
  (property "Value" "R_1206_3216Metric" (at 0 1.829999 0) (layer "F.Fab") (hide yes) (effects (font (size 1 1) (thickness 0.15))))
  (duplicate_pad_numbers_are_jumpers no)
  (fp_line (start -0.727064 0.91) (end 0.727064 0.91) (stroke (width 0.12) (type solid)) (layer "F.SilkS"))
  (fp_line (start -0.727064 -0.91) (end 0.727064 -0.91) (stroke (width 0.12) (type solid)) (layer "F.SilkS"))
  (pad "1" smd roundrect (at -1.4625 0 180) (size 1.125 1.75) (layers "F.Cu" "F.Mask" "F.Paste") (roundrect_rratio 0.222222))
  (pad "2" smd roundrect (at 1.4625 0 180) (size 1.125 1.75) (layers "F.Cu" "F.Mask" "F.Paste") (roundrect_rratio 0.222222)))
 (gr_rect (start 70.5 11.5) (end 120.5 96.5) (stroke (width 0.05) (type default)) (fill no) (layer "Edge.Cuts"))
 (segment (start 108.64 85.2) (end 108.64 79.23) (width 0.2) (layer "F.Cu") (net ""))
 (segment (start 81.14 61.2) (end 79.14 63.2) (width 0.2) (layer "F.Cu") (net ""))
 (segment (start 77.1775 87.2375) (end 76.64 86.7) (width 0.2) (layer "F.Cu") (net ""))
 (segment (start 82.14 88.199999) (end 80.1025 88.199999) (width 0.2) (layer "F.Cu") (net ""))
 (segment (start 115.7 79.7) (end 116.3 79.7) (width 0.2) (layer "F.Cu") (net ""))
 (segment (start 115.5 77.5) (end 113.6625 77.5) (width 0.2) (layer "F.Cu") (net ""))
 (segment (start 71 18) (end 71 59.5) (width 0.2) (layer "F.Cu") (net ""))
 (segment (start 115.699999 67.699999) (end 119 71) (width 0.2) (layer "F.Cu") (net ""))
 (segment (start 81.73 67.45) (end 81.64 67.36) (width 0.2) (layer "F.Cu") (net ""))
 (segment (start 85.54 64.8) (end 85.64 64.7) (width 0.2) (layer "F.Cu") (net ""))
 (segment (start 90.62 65.68) (end 89.64 64.7) (width 0.2) (layer "F.Cu") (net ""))
 (segment (start 79.14 63.2) (end 79.14 67.4) (width 0.2) (layer "F.Cu") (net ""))
 (segment (start 103.005 78.675) (end 103.005 81.335) (width 0.2) (layer "F.Cu") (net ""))
 (segment (start 91 12.5) (end 102.5 12.5) (width 0.2) (layer "F.Cu") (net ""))
 (segment (start 102.64 68.85) (end 102.64 70.2) (width 0.2) (layer "F.Cu") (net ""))
 (segment (start 107.64 86.2) (end 108.64 85.2) (width 0.2) (layer "F.Cu") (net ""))
 (segment (start 92.139999 62.7) (end 82.140001 62.7) (width 0.2) (layer "F.Cu") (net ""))
 (segment (start 77.1775 88.2) (end 77.1775 87.2375) (width 0.2) (layer "F.Cu") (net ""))
 (segment (start 110.5375 77.7) (end 109.5375 76.7) (width 0.2) (layer "F.Cu") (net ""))
 (segment (start 106.64 81.7) (end 106.64 78.85) (width 0.2) (layer "F.Cu") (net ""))
 (segment (start 110.037499 75.700001) (end 110.5375 75.2) (width 0.2) (layer "F.Cu") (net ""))
 (segment (start 99.64 76.7) (end 97.64 76.7) (width 0.2) (layer "F.Cu") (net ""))
 (segment (start 77.5 90) (end 77.5 88.5225) (width 0.2) (layer "F.Cu") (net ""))
 (segment (start 80.639999 67.27) (end 80.46 67.45) (width 0.2) (layer "F.Cu") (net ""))
 (segment (start 119 71) (end 119 83.84) (width 0.2) (layer "F.Cu") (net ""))
 (segment (start 82.140001 62.7) (end 80.64 64.200001) (width 0.2) (layer "F.Cu") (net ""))
 (segment (start 100.465 78.675) (end 100.464999 77.525) (width 0.2) (layer "F.Cu") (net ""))
 (segment (start 100.34 66.4) (end 93.64 59.7) (width 0.2) (layer "F.Cu") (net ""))
 (segment (start 115.5 75.5) (end 115.4025 75.5) (width 0.2) (layer "F.Cu") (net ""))
 (segment (start 106.64 86.2) (end 107.64 86.2) (width 0.2) (layer "F.Cu") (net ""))
 (segment (start 97.64 66.2) (end 92.64 61.2) (width 0.2) (layer "F.Cu") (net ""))
 (segment (start 109.5375 76.7) (end 105.64 76.7) (width 0.2) (layer "F.Cu") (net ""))
 (segment (start 102.64 70.2) (end 101.639999 71.2) (width 0.2) (layer "F.Cu") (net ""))
 (segment (start 93.64 59.7) (end 79.14 59.7) (width 0.2) (layer "F.Cu") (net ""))
 (segment (start 100.14 71.2) (end 99.195 72.145) (width 0.2) (layer "F.Cu") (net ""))
 (segment (start 77.92 86.0175) (end 77.92 84.95) (width 0.2) (layer "F.Cu") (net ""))
 (segment (start 103.005 81.335) (end 103.14 81.47) (width 0.2) (layer "F.Cu") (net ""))
 (segment (start 105.64 78.580001) (end 105.545 78.675) (width 0.2) (layer "F.Cu") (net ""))
 (segment (start 97.64 74.7) (end 97.64 66.2) (width 0.2) (layer "F.Cu") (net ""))
 (segment (start 103.14 81.47) (end 103.14 81.7) (width 0.2) (layer "F.Cu") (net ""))
 (segment (start 113.6625 77.5) (end 113.4625 77.7) (width 0.2) (layer "F.Cu") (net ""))
 (segment (start 91.89 64.95) (end 91.64 64.700001) (width 0.2) (layer "F.Cu") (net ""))
 (segment (start 75.17 63.67) (end 75.14 63.7) (width 0.2) (layer "F.Cu") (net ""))
 (segment (start 80.64 64.200001) (end 80.639999 67.27) (width 0.2) (layer "F.Cu") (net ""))
 (segment (start 91.89 67.45) (end 91.89 64.95) (width 0.2) (layer "F.Cu") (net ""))
 (segment (start 97.64 76.7) (end 96.14 75.2) (width 0.2) (layer "F.Cu") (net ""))
 (segment (start 119 28) (end 119 71) (width 0.2) (layer "F.Cu") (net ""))
 (segment (start 96.14 75.2) (end 96.14 66.700001) (width 0.2) (layer "F.Cu") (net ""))
 (segment (start 77.5 88.5225) (end 77.1775 88.2) (width 0.2) (layer "F.Cu") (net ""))
 (segment (start 101.639999 71.2) (end 100.14 71.2) (width 0.2) (layer "F.Cu") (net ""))
 (segment (start 102.5 12.5) (end 103.5 12.5) (width 0.2) (layer "F.Cu") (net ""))
 (segment (start 119 83.84) (end 112.14 90.7) (width 0.2) (layer "F.Cu") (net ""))
 (segment (start 89.5 14) (end 91 12.5) (width 0.2) (layer "F.Cu") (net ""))
 (segment (start 98.64 75.700001) (end 97.64 74.7) (width 0.2) (layer "F.Cu") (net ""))
 (segment (start 112.14 90.7) (end 78.2 90.7) (width 0.2) (layer "F.Cu") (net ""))
 (segment (start 104.275 78.675) (end 104.275 76.565) (width 0.2) (layer "F.Cu") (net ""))
 (segment (start 80.1025 88.199999) (end 77.92 86.0175) (width 0.2) (layer "F.Cu") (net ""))
 (segment (start 78.2 90.7) (end 77.5 90) (width 0.2) (layer "F.Cu") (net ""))
 (segment (start 92.64 61.2) (end 81.14 61.2) (width 0.2) (layer "F.Cu") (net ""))
 (segment (start 79.14 67.4) (end 79.19 67.45) (width 0.2) (layer "F.Cu") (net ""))
 (segment (start 76.65 86.69) (end 76.65 84.95) (width 0.2) (layer "F.Cu") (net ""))
 (segment (start 75.14 63.7) (end 75.14 67.21) (width 0.2) (layer "F.Cu") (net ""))
 (segment (start 110.14 67.699999) (end 115.699999 67.699999) (width 0.2) (layer "F.Cu") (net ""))
 (segment (start 105.64 76.7) (end 105.64 78.580001) (width 0.2) (layer "F.Cu") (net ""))
 (segment (start 79.2 93.7) (end 82.14 93.7) (width 0.2) (layer "F.Cu") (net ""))
 (segment (start 115.1025 75.2) (end 113.4625 75.2) (width 0.2) (layer "F.Cu") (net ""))
 (segment (start 100.14 75.7) (end 98.64 75.700001) (width 0.2) (layer "F.Cu") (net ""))
 (segment (start 100.464999 77.525) (end 99.64 76.7) (width 0.2) (layer "F.Cu") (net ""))
 (segment (start 115.5 79.5) (end 115.7 79.7) (width 0.2) (layer "F.Cu") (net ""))
 (segment (start 114.35 68.85) (end 104.94 68.85) (width 0.2) (layer "F.Cu") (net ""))
 (segment (start 104.275 76.565) (end 105.14 75.700001) (width 0.2) (layer "F.Cu") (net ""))
 (segment (start 84.27 67.45) (end 84.27 65.83) (width 0.2) (layer "F.Cu") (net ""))
 (segment (start 76 13) (end 86 13) (width 0.2) (layer "F.Cu") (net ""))
 (segment (start 117.5 72) (end 114.35 68.85) (width 0.2) (layer "F.Cu") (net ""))
 (segment (start 103.5 12.5) (end 119 28) (width 0.2) (layer "F.Cu") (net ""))
 (segment (start 99.14 78.73) (end 99.139999 81.2) (width 0.2) (layer "F.Cu") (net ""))
 (segment (start 85.54 67.45) (end 85.54 64.8) (width 0.2) (layer "F.Cu") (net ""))
 (segment (start 96.14 66.700001) (end 92.139999 62.7) (width 0.2) (layer "F.Cu") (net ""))
 (segment (start 105.14 81.7) (end 106.64 81.7) (width 0.2) (layer "F.Cu") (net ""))
 (segment (start 100.34 68.85) (end 100.34 66.4) (width 0.2) (layer "F.Cu") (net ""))
 (segment (start 71 59.5) (end 75.17 63.67) (width 0.2) (layer "F.Cu") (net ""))
 (segment (start 89.64 64.7) (end 88.14 64.7) (width 0.2) (layer "F.Cu") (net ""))
 (segment (start 117.5 78.5) (end 117.5 72.2) (width 0.2) (layer "F.Cu") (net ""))
 (segment (start 75.38 89.88) (end 79.2 93.7) (width 0.2) (layer "F.Cu") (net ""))
 (segment (start 101.735 77.294999) (end 100.14 75.7) (width 0.2) (layer "F.Cu") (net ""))
 (segment (start 76.64 64.7) (end 76.64 67.44) (width 0.2) (layer "F.Cu") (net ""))
 (segment (start 90.62 67.45) (end 90.62 65.68) (width 0.2) (layer "F.Cu") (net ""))
 (segment (start 73.5 15.5) (end 76 13) (width 0.2) (layer "F.Cu") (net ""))
 (segment (start 73.5 15.5) (end 71 18) (width 0.2) (layer "F.Cu") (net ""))
 (segment (start 101.735 78.675) (end 101.735 77.294999) (width 0.2) (layer "F.Cu") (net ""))
 (segment (start 86 13) (end 87 14) (width 0.2) (layer "F.Cu") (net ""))
 (segment (start 75.14 67.21) (end 75.38 67.45) (width 0.2) (layer "F.Cu") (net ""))
 (segment (start 76.64 67.44) (end 76.65 67.45) (width 0.2) (layer "F.Cu") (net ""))
 (segment (start 117.5 72.2) (end 117.5 72) (width 0.2) (layer "F.Cu") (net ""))
 (segment (start 99.139999 81.2) (end 98.425 81.915) (width 0.2) (layer "F.Cu") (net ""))
 (segment (start 105.14 86.2) (end 106.64 86.2) (width 0.2) (layer "F.Cu") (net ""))
 (segment (start 75.38 84.95) (end 75.38 89.88) (width 0.2) (layer "F.Cu") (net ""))
 (segment (start 79.14 59.7) (end 75.17 63.67) (width 0.2) (layer "F.Cu") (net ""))
 (segment (start 76.64 86.7) (end 76.65 86.69) (width 0.2) (layer "F.Cu") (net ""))
 (segment (start 104.99 62.549999) (end 110.14 67.699999) (width 0.2) (layer "F.Cu") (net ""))
 (segment (start 98.425 81.915) (end 93.14 81.915) (width 0.2) (layer "F.Cu") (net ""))
 (segment (start 99.14 81.7) (end 99.14 84.7) (width 0.2) (layer "F.Cu") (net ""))
 (segment (start 102.64 62.55) (end 104.99 62.549999) (width 0.2) (layer "F.Cu") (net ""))
 (segment (start 84.27 65.83) (end 83.14 64.7) (width 0.2) (layer "F.Cu") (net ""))
 (segment (start 116.3 79.7) (end 117.5 78.5) (width 0.2) (layer "F.Cu") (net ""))
 (segment (start 106.64 78.85) (end 106.815 78.675) (width 0.2) (layer "F.Cu") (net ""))
 (segment (start 99.195 72.145) (end 99.195 73.725) (width 0.2) (layer "F.Cu") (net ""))
 (segment (start 105.14 75.700001) (end 110.037499 75.700001) (width 0.2) (layer "F.Cu") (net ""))
 (segment (start 115.4025 75.5) (end 115.1025 75.2) (width 0.2) (layer "F.Cu") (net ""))
 (segment (start 99.195 78.675) (end 99.14 78.73) (width 0.2) (layer "F.Cu") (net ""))
 (segment (start 108.64 79.23) (end 108.085 78.675) (width 0.2) (layer "F.Cu") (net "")))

